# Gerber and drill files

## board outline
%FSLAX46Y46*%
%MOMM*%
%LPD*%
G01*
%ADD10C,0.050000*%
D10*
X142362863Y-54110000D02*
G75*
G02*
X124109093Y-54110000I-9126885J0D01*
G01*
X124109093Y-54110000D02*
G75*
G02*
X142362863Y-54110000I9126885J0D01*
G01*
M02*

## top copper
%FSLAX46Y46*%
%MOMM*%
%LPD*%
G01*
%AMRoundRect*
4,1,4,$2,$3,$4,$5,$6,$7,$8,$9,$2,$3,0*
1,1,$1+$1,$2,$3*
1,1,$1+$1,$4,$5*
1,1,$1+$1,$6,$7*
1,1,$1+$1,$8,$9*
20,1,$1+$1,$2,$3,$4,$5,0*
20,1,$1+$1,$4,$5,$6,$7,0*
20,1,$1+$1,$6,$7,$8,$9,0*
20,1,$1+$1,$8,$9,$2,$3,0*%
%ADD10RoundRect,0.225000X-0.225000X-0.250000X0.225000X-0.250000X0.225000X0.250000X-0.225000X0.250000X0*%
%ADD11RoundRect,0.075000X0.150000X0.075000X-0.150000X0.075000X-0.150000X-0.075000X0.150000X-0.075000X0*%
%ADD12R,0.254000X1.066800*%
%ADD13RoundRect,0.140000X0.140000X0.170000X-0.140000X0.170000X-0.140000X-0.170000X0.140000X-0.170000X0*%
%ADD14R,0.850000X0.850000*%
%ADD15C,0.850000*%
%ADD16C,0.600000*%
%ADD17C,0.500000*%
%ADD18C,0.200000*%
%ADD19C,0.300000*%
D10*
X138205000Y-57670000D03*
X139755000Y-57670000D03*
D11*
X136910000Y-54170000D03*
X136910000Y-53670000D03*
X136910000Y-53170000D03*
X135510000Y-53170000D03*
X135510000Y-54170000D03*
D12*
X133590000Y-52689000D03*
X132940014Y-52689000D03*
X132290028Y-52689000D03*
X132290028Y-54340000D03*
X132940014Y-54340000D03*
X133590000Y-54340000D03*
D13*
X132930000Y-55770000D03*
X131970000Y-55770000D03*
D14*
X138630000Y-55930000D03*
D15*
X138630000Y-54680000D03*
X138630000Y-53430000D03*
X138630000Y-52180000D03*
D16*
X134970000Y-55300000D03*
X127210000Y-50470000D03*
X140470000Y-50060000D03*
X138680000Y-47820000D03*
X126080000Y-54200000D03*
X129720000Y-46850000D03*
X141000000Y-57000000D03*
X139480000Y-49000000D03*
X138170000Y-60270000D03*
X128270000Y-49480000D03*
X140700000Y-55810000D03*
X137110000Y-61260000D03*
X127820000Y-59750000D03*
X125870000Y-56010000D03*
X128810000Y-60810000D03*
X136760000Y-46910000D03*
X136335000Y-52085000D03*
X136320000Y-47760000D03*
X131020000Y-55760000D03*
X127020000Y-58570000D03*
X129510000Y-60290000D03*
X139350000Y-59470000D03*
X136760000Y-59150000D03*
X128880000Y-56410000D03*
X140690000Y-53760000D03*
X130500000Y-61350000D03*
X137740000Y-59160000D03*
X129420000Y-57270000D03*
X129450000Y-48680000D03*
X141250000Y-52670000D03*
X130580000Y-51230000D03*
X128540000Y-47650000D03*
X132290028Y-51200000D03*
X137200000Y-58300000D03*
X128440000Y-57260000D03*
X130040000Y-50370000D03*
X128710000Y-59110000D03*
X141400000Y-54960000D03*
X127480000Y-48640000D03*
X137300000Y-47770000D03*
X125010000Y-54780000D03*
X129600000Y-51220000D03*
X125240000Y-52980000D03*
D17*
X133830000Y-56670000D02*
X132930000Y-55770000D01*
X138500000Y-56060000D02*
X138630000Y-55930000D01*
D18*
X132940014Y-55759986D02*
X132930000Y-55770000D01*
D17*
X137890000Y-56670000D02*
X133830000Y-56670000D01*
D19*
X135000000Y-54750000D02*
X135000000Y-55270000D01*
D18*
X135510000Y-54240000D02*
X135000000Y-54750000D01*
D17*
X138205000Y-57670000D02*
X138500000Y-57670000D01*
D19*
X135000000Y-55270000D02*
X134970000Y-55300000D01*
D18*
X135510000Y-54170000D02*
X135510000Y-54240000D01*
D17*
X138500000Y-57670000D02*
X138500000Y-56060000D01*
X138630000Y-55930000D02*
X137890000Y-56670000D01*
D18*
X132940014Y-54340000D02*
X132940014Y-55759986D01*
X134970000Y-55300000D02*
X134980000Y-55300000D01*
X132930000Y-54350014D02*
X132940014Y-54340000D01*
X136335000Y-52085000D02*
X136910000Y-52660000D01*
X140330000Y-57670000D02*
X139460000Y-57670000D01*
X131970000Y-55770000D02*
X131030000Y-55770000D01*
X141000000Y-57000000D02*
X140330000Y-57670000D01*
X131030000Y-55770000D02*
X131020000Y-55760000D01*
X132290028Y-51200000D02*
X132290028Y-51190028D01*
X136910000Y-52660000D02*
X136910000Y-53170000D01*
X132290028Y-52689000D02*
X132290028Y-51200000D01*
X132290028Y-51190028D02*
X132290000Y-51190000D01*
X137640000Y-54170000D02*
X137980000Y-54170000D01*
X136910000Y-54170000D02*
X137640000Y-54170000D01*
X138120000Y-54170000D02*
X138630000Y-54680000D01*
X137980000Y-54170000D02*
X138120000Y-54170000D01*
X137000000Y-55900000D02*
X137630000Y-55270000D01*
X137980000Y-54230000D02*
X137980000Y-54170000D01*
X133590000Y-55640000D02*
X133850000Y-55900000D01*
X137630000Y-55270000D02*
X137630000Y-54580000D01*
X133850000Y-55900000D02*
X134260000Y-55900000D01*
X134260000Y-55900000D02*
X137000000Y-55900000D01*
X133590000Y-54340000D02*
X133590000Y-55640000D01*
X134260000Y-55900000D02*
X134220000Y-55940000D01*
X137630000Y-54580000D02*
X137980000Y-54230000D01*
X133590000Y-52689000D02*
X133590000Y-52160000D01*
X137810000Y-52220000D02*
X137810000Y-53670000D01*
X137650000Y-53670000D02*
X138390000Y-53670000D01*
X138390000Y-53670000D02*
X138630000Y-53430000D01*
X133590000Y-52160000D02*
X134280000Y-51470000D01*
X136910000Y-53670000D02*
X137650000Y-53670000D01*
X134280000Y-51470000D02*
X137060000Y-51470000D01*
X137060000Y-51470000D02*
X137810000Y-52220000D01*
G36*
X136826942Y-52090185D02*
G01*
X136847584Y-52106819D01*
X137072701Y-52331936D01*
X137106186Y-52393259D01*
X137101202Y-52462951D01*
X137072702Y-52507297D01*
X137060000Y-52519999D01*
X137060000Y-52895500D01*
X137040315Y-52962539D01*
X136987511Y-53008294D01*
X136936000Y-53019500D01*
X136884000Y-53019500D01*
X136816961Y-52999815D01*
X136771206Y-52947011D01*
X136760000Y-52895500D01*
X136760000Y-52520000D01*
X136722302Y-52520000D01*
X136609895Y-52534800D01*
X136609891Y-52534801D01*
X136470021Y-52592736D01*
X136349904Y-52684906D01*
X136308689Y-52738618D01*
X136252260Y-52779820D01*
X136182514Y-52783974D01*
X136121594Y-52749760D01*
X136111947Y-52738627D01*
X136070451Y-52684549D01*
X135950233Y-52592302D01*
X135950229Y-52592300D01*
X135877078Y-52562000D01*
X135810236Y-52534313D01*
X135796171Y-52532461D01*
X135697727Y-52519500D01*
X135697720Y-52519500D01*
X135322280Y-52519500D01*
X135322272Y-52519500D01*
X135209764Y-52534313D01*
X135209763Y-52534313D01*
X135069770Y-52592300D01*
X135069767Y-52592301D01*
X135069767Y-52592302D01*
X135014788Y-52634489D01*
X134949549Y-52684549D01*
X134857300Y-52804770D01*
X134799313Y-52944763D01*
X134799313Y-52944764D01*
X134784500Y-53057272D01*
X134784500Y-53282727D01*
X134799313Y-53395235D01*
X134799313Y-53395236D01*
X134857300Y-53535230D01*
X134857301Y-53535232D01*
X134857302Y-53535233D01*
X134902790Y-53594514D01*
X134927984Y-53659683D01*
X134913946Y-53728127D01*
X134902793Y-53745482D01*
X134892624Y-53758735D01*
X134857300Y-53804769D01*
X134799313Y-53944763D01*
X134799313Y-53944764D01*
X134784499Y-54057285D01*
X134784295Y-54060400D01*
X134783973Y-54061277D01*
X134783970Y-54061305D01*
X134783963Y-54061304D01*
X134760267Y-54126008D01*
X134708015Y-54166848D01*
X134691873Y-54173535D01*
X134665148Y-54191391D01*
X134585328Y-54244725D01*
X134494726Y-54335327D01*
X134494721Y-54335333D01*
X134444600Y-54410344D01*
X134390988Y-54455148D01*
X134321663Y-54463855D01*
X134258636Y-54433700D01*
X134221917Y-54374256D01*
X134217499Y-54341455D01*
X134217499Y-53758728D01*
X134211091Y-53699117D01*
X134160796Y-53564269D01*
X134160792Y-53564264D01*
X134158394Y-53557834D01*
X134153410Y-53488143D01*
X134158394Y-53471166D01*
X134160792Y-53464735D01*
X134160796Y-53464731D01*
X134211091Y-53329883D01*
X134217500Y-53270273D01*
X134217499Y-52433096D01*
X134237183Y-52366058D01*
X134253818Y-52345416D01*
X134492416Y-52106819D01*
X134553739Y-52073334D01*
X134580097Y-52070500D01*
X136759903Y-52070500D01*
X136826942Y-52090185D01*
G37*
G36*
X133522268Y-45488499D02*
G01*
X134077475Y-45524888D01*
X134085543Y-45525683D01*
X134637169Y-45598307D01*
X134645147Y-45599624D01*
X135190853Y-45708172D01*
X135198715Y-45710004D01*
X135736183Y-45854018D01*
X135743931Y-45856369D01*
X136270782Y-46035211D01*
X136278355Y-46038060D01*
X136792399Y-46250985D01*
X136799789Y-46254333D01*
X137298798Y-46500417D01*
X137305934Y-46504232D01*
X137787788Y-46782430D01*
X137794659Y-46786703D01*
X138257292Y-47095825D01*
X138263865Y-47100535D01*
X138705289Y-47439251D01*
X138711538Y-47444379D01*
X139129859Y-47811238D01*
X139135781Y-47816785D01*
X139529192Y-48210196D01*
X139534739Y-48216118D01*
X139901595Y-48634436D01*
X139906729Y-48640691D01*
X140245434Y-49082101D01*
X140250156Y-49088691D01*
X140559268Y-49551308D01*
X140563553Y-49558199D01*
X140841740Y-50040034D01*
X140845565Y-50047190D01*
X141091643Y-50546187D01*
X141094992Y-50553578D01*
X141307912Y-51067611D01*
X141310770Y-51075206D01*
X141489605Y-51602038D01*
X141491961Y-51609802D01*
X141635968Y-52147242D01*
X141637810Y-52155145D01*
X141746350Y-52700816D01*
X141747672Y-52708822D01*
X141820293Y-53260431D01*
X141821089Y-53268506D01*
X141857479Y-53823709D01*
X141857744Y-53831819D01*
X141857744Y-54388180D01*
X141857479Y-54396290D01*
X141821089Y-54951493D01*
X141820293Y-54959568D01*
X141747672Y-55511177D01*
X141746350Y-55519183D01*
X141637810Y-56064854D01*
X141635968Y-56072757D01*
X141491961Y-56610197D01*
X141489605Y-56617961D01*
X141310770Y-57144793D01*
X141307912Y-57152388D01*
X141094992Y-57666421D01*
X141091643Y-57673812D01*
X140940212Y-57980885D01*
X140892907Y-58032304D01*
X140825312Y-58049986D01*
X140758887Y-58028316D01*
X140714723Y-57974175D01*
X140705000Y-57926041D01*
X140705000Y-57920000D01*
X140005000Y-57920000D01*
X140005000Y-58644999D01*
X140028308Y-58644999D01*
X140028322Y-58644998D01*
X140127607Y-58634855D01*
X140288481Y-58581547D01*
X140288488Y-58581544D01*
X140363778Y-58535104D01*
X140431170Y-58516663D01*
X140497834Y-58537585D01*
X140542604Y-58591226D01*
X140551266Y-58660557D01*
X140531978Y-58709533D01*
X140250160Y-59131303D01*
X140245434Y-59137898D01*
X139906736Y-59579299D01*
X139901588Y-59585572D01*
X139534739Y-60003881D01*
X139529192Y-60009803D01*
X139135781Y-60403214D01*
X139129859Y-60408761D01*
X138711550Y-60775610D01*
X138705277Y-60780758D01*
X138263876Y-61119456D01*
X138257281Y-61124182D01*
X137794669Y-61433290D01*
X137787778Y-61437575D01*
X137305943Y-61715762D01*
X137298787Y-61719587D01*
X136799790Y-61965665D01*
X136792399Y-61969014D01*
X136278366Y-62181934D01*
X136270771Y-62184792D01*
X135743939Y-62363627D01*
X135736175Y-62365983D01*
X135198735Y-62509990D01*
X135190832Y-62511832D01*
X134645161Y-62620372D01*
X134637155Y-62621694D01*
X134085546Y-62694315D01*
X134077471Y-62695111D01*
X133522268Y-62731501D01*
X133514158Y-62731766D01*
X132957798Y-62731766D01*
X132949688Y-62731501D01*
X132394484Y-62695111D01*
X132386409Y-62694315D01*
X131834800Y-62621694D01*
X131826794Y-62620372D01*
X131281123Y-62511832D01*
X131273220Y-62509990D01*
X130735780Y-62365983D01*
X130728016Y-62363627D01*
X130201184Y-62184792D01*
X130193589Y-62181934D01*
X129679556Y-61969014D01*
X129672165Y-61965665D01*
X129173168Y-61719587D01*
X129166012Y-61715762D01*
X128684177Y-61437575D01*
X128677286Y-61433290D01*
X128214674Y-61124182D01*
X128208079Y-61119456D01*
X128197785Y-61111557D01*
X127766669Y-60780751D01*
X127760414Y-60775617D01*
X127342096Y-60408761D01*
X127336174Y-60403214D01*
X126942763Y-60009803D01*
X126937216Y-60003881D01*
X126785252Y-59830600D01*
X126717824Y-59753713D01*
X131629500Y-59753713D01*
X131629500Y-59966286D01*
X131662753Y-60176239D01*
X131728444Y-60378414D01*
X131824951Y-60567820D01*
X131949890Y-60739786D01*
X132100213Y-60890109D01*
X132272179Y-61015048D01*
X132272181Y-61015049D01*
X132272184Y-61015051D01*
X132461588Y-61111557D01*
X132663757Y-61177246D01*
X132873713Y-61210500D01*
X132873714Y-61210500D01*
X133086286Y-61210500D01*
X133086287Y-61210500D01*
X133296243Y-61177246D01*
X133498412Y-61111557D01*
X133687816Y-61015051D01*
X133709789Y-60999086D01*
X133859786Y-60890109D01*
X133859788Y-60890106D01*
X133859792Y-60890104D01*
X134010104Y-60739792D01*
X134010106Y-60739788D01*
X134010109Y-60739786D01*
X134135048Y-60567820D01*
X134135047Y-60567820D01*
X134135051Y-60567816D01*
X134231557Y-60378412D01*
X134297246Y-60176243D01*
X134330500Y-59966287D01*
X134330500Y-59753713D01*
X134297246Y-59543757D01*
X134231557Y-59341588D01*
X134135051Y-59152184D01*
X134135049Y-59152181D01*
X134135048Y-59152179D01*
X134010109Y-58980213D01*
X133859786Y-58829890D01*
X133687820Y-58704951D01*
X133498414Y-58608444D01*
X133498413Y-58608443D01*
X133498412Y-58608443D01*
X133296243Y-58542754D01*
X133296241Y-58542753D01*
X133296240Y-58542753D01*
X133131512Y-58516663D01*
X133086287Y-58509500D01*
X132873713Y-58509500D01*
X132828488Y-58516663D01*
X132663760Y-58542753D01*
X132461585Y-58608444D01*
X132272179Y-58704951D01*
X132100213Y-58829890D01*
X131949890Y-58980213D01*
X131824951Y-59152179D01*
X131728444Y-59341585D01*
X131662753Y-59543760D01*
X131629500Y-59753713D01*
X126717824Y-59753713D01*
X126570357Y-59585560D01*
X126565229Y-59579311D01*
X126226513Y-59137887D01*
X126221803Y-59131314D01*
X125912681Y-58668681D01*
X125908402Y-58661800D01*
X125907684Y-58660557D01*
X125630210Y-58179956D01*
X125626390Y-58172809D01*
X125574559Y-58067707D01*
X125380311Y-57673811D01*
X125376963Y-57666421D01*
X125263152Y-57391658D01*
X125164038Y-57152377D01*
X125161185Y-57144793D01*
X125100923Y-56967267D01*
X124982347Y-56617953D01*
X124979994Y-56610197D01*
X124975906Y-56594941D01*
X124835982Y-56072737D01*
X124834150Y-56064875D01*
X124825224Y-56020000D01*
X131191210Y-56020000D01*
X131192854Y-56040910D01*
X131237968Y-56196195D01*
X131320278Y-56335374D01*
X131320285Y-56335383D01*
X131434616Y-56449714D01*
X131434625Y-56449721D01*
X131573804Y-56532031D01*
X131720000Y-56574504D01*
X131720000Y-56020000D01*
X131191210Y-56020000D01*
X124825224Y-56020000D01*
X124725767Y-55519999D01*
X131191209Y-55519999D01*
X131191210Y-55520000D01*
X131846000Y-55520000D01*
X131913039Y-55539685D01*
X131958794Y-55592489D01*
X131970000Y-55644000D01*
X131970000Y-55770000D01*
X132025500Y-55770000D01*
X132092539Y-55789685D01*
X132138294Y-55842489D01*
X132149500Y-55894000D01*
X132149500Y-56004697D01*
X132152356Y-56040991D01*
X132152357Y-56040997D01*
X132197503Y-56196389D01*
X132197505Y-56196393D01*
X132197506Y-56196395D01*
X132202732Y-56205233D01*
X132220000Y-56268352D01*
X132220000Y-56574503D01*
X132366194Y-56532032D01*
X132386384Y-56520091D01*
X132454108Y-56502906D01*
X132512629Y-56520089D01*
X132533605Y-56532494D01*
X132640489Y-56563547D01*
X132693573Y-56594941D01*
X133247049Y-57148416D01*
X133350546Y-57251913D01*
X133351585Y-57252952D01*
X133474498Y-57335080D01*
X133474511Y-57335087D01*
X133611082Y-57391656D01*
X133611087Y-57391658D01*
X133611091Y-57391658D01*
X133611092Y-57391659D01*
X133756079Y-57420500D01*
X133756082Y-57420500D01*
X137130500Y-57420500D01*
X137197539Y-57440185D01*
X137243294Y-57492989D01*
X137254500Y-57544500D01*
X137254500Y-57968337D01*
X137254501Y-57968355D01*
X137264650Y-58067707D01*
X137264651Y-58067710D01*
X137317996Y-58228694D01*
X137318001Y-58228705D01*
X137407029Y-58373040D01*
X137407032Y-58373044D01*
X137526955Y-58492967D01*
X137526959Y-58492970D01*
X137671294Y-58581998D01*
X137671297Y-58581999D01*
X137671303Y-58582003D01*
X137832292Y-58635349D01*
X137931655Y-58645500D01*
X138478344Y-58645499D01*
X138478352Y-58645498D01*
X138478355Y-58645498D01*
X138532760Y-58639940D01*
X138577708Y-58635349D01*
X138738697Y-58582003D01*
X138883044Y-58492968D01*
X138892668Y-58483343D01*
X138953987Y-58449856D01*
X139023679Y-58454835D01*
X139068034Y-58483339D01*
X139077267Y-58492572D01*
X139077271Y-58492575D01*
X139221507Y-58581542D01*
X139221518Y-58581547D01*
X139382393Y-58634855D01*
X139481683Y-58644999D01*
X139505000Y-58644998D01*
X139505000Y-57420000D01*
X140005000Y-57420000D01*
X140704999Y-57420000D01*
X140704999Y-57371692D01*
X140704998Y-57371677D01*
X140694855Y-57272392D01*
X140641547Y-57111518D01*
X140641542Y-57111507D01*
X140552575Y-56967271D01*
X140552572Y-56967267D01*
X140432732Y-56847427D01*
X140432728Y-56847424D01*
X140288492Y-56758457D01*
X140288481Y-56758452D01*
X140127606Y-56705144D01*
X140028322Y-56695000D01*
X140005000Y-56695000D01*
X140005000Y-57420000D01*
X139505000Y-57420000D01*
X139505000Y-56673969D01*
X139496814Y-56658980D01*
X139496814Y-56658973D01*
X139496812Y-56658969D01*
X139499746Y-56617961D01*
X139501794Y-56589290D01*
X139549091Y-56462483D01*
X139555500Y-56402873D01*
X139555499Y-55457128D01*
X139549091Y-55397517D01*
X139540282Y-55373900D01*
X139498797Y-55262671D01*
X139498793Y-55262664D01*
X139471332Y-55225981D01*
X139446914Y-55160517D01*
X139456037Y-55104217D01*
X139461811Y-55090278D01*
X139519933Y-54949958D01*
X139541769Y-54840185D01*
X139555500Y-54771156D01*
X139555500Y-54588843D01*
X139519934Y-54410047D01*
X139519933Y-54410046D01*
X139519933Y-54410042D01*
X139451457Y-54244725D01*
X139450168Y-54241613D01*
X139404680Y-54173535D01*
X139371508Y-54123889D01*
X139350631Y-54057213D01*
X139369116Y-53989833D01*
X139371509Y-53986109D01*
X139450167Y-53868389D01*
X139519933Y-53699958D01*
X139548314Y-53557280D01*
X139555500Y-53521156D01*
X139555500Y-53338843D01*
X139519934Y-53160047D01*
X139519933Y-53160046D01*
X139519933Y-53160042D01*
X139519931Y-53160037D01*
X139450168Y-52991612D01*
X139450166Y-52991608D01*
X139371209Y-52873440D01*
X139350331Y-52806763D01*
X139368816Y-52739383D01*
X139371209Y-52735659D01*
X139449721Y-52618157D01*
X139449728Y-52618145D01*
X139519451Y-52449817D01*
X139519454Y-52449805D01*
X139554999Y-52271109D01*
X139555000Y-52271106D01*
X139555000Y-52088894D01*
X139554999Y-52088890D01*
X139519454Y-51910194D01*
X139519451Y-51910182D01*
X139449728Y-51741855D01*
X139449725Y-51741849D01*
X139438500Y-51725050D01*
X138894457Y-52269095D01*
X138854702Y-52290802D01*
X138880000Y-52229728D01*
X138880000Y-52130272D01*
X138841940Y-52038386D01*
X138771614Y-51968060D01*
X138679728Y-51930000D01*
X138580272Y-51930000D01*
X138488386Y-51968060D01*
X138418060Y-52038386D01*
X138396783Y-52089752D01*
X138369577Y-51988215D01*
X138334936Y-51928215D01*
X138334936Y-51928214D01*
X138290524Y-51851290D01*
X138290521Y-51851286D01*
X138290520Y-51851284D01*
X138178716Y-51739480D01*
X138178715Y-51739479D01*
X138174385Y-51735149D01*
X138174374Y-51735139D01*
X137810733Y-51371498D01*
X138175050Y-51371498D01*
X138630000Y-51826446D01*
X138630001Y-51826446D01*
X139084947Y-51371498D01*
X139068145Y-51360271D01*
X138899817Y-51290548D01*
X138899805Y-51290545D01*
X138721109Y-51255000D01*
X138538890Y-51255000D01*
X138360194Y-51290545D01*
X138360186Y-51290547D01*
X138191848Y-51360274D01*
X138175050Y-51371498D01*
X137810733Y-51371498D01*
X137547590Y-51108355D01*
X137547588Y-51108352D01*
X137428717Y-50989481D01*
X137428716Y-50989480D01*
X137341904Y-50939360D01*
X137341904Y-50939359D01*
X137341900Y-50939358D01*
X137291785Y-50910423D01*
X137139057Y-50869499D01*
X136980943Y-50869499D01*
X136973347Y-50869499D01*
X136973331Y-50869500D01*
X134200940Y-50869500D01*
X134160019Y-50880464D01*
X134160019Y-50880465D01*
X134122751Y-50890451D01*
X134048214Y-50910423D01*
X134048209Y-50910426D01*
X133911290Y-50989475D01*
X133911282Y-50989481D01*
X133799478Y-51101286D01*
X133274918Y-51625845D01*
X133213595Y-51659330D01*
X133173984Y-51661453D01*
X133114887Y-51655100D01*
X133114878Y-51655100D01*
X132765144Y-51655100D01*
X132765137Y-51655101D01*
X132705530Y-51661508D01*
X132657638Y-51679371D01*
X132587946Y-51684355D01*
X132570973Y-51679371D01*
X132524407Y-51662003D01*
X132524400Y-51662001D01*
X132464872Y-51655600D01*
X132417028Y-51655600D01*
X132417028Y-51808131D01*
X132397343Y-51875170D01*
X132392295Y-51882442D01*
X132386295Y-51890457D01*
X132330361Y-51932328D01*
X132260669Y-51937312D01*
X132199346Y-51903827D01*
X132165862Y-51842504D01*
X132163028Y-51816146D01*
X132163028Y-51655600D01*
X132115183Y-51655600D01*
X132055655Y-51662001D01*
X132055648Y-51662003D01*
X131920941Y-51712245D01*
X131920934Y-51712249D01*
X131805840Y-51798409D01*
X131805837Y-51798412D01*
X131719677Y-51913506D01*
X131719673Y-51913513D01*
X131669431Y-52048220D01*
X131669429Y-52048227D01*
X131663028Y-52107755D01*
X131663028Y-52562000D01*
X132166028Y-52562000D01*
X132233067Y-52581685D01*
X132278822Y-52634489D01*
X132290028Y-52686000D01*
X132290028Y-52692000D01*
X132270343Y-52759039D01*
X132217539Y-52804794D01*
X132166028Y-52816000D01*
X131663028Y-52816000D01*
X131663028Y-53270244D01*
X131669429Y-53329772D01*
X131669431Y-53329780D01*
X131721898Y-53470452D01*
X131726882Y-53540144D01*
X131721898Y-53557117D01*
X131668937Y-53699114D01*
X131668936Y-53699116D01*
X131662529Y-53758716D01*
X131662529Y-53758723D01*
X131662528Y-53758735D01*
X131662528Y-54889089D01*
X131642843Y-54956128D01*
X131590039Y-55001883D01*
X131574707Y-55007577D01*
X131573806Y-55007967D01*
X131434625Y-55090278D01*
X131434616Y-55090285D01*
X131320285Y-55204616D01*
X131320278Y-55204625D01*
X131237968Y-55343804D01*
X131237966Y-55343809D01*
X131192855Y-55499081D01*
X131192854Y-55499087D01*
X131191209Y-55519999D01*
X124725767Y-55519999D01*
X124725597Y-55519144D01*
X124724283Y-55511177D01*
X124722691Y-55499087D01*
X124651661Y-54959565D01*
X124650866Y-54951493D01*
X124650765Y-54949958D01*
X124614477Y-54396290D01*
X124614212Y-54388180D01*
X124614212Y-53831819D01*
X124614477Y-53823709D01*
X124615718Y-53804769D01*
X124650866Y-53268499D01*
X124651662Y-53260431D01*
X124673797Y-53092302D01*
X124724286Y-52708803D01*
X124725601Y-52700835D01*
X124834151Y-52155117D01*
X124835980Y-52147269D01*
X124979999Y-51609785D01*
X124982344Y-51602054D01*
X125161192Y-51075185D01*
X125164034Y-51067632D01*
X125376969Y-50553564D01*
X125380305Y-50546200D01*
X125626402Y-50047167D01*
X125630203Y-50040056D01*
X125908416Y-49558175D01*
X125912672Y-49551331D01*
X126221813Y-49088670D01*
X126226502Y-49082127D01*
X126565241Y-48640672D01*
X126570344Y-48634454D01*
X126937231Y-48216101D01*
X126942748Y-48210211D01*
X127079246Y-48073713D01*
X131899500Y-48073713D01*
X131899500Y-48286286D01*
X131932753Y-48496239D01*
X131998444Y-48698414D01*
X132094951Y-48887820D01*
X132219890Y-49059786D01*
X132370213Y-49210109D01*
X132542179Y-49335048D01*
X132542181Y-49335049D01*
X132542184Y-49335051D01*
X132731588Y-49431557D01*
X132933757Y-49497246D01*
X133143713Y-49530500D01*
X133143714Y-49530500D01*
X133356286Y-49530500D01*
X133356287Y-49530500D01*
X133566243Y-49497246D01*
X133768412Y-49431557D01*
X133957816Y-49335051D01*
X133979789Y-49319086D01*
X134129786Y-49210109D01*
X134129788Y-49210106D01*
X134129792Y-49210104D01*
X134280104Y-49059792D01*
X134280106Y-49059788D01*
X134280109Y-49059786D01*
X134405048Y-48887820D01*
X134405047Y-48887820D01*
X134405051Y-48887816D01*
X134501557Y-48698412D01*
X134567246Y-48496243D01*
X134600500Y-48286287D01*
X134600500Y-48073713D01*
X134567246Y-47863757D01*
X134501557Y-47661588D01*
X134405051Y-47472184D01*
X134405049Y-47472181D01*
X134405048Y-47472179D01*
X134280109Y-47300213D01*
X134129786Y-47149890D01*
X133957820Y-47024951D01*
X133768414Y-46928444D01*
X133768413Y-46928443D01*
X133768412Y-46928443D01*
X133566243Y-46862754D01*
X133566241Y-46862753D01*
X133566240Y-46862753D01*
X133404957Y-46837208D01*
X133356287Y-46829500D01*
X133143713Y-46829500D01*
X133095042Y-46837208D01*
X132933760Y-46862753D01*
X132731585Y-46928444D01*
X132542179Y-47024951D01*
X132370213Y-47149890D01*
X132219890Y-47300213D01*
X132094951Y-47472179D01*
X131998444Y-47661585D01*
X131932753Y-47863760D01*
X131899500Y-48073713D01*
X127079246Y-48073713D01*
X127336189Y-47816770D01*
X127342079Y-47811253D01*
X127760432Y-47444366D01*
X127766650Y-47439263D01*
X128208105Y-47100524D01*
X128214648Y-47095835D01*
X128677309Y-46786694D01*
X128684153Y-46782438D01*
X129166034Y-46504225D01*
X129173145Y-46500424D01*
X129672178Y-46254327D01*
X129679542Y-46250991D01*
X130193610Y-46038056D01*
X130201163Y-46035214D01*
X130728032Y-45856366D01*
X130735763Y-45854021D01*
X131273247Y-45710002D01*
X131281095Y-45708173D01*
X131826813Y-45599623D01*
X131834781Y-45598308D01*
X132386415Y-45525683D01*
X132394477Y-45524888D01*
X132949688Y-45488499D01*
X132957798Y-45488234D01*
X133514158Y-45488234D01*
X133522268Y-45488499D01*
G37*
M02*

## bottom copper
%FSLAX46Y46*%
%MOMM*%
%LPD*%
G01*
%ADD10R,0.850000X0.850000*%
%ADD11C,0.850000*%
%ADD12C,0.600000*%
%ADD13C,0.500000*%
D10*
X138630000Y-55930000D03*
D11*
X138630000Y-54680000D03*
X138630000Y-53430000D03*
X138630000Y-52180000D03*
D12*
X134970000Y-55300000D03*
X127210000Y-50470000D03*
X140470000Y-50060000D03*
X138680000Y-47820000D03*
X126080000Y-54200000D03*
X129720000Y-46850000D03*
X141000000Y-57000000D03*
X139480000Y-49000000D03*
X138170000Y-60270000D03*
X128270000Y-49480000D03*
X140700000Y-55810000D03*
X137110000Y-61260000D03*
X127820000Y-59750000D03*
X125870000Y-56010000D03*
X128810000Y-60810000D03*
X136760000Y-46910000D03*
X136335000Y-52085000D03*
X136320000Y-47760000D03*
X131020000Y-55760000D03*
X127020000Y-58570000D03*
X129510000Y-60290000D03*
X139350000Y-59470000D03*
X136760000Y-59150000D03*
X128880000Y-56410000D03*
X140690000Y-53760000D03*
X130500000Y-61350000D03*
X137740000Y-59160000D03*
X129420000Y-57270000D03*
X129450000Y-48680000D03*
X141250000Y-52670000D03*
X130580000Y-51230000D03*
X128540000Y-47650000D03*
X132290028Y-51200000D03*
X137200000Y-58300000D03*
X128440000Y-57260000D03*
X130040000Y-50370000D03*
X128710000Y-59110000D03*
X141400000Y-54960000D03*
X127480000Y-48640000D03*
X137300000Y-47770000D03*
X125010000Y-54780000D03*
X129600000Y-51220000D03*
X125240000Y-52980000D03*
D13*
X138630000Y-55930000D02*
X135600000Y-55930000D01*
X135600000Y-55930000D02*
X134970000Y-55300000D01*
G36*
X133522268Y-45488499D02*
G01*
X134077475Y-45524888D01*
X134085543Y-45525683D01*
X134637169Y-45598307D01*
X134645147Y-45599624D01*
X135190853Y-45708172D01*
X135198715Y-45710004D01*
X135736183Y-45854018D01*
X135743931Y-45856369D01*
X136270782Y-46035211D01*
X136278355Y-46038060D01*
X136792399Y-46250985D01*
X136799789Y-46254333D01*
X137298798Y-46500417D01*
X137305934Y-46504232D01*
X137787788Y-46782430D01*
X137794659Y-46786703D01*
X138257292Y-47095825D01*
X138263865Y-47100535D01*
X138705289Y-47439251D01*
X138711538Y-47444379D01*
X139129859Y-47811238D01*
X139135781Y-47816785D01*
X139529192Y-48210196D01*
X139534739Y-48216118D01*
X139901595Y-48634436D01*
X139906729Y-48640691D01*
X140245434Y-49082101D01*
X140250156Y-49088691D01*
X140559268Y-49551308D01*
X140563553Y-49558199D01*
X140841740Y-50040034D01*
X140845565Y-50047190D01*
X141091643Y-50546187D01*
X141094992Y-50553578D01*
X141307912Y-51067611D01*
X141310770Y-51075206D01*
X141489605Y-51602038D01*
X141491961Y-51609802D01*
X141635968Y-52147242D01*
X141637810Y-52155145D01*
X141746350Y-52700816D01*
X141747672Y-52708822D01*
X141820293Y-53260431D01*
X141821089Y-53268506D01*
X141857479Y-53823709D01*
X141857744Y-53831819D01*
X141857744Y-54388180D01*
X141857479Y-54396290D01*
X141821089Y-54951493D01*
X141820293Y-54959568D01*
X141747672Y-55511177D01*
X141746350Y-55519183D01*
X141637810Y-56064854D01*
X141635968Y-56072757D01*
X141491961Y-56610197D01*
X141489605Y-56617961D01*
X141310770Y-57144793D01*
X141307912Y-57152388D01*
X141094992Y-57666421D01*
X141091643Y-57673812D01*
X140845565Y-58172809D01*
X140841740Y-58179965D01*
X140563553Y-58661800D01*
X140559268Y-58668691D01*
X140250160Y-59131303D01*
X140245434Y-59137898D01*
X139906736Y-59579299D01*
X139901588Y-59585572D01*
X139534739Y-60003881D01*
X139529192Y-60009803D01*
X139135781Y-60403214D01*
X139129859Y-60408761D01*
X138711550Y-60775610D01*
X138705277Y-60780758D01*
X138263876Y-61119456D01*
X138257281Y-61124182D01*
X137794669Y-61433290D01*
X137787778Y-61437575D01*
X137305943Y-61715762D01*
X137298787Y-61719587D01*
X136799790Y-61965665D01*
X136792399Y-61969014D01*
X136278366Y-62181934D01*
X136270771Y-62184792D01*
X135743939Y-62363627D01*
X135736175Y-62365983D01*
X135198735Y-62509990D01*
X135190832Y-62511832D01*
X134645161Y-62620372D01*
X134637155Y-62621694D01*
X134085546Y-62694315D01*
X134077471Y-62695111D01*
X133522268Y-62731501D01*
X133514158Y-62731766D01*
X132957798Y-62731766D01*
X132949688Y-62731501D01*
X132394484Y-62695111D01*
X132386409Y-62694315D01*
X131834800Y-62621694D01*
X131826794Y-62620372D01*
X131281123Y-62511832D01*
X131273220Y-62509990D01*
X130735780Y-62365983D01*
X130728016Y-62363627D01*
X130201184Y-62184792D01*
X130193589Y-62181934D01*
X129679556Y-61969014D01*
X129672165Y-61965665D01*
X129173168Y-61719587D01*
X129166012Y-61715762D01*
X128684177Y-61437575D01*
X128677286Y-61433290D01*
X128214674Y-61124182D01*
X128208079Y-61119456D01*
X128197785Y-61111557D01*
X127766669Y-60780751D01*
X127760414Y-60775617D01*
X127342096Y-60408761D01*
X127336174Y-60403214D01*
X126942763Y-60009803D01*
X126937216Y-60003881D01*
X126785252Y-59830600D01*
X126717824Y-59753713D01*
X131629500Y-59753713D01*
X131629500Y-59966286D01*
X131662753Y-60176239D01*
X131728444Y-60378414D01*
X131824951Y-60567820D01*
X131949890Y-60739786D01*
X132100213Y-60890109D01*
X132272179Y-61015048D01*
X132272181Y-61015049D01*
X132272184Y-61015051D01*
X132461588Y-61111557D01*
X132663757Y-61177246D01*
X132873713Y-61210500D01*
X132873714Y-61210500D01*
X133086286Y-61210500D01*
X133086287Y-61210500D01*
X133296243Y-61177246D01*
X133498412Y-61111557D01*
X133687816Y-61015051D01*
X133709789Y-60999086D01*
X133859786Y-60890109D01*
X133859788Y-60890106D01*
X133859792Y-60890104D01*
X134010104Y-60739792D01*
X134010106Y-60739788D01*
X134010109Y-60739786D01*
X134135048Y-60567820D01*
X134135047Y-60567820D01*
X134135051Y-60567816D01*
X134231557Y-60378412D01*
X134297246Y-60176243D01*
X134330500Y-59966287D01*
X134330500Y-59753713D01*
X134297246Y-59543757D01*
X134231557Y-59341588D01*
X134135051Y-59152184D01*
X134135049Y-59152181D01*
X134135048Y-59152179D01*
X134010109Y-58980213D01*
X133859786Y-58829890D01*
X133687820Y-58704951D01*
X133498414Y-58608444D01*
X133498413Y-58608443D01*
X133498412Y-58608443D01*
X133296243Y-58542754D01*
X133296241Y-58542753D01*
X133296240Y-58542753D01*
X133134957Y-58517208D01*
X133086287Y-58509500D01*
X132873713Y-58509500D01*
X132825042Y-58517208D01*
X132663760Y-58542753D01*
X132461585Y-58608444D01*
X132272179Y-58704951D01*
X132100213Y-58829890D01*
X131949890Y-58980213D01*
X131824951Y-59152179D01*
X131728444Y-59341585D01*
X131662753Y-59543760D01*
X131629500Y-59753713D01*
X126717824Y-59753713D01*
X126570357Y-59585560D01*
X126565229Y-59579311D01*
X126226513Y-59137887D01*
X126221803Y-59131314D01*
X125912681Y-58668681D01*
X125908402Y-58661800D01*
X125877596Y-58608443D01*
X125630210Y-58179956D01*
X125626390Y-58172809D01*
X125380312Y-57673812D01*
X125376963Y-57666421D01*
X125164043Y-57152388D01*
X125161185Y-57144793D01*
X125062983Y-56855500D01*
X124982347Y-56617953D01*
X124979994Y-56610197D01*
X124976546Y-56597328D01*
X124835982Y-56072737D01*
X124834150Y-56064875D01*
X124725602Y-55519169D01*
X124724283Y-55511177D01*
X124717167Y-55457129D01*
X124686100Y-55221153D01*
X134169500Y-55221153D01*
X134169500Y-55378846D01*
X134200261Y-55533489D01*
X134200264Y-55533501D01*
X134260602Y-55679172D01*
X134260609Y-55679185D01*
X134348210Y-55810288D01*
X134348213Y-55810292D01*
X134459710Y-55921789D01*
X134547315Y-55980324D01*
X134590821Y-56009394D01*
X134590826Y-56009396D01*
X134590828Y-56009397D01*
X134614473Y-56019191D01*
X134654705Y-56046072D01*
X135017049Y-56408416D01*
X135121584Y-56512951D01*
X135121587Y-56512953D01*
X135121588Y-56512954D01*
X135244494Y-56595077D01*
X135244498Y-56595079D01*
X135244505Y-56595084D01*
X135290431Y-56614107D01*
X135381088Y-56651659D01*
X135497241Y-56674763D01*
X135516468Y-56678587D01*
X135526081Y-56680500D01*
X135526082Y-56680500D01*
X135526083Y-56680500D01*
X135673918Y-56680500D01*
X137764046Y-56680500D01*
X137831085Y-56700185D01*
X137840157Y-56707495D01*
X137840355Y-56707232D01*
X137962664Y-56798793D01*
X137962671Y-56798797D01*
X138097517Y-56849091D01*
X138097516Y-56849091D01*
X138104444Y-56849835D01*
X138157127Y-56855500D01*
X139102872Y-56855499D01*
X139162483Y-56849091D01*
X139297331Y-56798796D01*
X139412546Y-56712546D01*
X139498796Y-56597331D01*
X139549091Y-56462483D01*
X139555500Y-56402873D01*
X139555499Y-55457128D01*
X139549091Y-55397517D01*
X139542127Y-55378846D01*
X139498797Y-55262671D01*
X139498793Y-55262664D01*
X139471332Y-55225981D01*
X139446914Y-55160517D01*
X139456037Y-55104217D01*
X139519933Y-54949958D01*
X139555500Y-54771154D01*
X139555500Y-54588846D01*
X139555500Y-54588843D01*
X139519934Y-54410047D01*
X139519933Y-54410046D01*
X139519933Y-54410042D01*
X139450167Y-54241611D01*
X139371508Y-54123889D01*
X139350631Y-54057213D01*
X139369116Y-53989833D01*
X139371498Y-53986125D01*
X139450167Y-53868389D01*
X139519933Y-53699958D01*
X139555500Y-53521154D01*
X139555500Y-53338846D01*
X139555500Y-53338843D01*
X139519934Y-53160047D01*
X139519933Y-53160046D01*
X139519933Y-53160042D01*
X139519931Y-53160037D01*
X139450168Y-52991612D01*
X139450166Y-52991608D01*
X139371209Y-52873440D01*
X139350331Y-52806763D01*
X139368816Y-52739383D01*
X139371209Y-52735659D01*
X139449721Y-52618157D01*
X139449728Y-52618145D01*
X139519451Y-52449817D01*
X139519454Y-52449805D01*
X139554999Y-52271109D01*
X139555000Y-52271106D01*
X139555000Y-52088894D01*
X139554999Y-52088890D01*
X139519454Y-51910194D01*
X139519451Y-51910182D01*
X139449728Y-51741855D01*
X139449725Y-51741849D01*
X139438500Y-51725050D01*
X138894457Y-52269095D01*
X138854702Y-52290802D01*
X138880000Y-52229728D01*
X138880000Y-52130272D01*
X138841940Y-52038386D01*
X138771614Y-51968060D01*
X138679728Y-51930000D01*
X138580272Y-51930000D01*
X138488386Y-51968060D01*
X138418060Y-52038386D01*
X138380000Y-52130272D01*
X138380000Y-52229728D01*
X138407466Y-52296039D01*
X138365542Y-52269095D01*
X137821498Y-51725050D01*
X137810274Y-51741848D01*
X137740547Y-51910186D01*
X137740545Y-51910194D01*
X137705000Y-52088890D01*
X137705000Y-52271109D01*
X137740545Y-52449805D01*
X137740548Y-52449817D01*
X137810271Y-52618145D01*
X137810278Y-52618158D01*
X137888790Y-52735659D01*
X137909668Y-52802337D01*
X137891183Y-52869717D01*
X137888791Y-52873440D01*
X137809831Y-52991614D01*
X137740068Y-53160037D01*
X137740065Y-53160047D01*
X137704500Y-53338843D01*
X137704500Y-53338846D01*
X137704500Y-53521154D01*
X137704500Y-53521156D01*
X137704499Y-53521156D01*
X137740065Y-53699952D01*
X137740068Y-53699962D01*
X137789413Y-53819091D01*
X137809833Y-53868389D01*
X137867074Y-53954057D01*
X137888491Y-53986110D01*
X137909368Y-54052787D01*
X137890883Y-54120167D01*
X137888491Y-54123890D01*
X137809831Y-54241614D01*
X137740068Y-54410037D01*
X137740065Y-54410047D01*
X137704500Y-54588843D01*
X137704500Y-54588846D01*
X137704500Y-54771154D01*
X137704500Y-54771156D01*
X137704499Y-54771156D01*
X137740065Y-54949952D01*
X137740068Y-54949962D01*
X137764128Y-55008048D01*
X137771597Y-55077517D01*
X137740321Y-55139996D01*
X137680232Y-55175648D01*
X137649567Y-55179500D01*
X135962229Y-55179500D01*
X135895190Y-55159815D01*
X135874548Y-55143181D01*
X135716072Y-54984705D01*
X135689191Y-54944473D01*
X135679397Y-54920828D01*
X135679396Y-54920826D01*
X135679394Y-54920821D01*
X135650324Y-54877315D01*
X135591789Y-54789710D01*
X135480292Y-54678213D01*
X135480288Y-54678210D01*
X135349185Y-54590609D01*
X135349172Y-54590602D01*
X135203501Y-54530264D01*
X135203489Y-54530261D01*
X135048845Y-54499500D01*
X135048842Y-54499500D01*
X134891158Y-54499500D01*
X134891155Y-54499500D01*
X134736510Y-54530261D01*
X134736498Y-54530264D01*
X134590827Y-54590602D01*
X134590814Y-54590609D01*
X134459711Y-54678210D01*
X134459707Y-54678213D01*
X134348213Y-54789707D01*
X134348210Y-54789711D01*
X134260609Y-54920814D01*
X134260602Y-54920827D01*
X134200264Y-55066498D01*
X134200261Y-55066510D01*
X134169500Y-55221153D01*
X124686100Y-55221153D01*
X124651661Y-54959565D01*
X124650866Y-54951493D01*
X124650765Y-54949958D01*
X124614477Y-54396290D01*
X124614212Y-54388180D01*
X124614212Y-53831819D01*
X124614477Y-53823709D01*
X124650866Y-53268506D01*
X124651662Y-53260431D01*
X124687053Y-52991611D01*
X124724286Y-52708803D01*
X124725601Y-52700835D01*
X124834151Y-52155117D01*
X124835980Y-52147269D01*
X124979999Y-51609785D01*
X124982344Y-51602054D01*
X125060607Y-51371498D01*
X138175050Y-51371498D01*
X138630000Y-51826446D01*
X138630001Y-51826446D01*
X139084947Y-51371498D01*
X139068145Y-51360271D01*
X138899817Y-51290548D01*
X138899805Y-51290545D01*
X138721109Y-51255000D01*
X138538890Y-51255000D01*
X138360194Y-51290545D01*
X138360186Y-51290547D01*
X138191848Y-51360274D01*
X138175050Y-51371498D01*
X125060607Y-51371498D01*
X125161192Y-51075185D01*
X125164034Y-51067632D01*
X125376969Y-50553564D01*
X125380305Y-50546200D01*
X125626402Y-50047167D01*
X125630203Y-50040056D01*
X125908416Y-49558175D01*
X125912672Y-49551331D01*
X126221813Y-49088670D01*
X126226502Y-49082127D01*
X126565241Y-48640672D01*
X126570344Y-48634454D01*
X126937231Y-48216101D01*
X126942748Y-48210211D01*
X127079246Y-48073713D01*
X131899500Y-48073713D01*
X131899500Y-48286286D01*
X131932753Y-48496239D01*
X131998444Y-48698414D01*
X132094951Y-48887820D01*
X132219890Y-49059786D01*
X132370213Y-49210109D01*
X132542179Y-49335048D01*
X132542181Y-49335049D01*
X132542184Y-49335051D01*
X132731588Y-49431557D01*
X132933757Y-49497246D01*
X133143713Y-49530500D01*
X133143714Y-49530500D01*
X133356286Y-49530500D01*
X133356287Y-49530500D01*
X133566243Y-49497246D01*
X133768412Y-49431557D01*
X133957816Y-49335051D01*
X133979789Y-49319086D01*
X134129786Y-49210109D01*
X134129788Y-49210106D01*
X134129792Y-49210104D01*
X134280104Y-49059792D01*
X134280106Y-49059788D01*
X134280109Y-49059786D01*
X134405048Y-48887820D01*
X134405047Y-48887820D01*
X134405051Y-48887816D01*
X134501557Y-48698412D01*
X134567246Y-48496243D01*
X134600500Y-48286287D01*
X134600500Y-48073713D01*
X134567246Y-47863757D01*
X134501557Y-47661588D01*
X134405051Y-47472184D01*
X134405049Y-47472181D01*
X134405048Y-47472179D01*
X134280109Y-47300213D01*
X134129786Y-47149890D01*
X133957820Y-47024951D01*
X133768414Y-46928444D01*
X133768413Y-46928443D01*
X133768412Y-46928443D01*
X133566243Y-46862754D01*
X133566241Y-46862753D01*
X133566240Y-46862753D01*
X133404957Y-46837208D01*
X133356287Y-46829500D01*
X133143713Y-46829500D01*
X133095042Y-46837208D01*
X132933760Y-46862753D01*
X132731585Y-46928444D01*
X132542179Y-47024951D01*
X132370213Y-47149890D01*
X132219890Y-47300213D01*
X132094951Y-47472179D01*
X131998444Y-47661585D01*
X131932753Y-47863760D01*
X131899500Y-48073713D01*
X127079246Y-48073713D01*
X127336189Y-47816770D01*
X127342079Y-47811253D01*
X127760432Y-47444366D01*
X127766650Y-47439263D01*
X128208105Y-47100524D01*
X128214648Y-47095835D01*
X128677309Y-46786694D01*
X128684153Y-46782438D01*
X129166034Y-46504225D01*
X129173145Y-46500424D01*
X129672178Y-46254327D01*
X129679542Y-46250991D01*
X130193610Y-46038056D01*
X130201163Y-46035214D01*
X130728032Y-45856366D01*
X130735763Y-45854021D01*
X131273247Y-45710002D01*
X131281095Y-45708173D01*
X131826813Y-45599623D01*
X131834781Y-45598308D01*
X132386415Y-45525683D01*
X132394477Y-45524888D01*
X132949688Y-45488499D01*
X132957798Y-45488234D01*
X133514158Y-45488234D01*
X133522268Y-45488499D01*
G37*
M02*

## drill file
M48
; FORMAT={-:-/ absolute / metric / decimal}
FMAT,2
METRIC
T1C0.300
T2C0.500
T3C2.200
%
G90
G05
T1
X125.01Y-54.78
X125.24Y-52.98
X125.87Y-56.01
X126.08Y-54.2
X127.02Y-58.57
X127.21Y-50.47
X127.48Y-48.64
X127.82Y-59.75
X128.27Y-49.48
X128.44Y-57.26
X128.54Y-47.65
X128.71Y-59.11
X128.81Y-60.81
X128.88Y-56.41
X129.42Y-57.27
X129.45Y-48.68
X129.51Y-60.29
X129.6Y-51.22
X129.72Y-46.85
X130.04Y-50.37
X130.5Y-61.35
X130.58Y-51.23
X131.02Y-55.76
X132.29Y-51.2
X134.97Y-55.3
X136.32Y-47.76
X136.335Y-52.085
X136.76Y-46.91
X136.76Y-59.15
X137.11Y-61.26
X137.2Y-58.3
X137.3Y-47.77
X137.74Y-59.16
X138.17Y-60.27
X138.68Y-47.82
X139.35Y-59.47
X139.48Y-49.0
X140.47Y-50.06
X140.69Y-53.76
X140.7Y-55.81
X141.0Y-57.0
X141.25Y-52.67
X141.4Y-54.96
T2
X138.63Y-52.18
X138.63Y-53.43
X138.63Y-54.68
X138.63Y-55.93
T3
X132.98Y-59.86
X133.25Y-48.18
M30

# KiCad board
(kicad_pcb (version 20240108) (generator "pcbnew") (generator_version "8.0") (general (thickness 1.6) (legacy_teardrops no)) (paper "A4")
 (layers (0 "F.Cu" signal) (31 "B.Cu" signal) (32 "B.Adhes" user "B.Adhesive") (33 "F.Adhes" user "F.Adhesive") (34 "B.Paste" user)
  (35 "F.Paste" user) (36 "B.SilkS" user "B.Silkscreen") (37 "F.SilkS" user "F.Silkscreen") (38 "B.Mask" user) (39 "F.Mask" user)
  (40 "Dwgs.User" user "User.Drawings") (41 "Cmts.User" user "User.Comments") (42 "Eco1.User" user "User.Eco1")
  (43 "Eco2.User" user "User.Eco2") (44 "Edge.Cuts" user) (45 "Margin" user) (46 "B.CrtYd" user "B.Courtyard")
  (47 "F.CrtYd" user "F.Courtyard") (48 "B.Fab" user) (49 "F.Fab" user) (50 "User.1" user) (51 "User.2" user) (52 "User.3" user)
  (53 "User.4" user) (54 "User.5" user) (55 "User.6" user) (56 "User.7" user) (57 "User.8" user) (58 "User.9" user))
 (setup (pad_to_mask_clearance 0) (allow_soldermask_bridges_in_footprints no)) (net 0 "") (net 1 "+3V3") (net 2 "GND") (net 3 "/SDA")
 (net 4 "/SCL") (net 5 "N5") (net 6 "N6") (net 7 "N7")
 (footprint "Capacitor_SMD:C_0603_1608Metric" (layer "F.Cu") (at 138.98 57.67)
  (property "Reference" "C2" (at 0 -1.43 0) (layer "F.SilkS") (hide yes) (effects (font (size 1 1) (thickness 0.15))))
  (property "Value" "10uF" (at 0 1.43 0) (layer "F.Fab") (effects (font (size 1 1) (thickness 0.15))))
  (pad "1" smd roundrect (at -0.775 0) (size 0.9 0.95) (layers "F.Cu" "F.Paste" "F.Mask") (roundrect_rratio 0.25) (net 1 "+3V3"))
  (pad "2" smd roundrect (at 0.775 0) (size 0.9 0.95) (layers "F.Cu" "F.Paste" "F.Mask") (roundrect_rratio 0.25) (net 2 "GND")))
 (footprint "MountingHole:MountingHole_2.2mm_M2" (layer "F.Cu") (at 132.98 59.86)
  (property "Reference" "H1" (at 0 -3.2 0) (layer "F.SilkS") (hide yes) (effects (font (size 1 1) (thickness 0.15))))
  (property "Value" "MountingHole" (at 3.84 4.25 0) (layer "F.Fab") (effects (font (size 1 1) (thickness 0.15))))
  (pad "" np_thru_hole circle (at 0 0) (size 2.2 2.2) (drill 2.2) (layers "*.Cu" "*.Mask")))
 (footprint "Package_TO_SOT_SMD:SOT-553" (layer "F.Cu") (at 136.21 53.67 180)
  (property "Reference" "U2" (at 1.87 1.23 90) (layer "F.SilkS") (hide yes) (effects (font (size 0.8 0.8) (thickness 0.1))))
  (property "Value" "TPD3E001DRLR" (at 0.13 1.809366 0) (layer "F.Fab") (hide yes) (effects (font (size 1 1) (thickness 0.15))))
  (pad "1" smd roundrect (at -0.7 -0.5 180) (size 0.45 0.3) (layers "F.Cu" "F.Paste" "F.Mask") (roundrect_rratio 0.25) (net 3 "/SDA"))
  (pad "2" smd roundrect (at -0.7 0 180) (size 0.45 0.3) (layers "F.Cu" "F.Paste" "F.Mask") (roundrect_rratio 0.25) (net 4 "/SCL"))
  (pad "3" smd roundrect (at -0.7 0.5 180) (size 0.45 0.3) (layers "F.Cu" "F.Paste" "F.Mask") (roundrect_rratio 0.25) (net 2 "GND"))
  (pad "4" smd roundrect (at 0.7 0.5 180) (size 0.45 0.3) (layers "F.Cu" "F.Paste" "F.Mask") (roundrect_rratio 0.25) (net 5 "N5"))
  (pad "5" smd roundrect (at 0.7 -0.5 180) (size 0.45 0.3) (layers "F.Cu" "F.Paste" "F.Mask") (roundrect_rratio 0.25) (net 1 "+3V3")))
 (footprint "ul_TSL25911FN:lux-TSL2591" (layer "F.Cu") (at 132.940014 53.5145 -90)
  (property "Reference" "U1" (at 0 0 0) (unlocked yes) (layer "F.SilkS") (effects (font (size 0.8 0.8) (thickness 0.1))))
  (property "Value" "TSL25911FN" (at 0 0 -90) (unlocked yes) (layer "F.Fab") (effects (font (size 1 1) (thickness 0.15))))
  (pad "1" smd rect (at -0.8255 -0.649986 270) (size 1.0668 0.254) (layers "F.Cu" "F.Paste" "F.Mask") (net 4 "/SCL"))
  (pad "2" smd rect (at -0.8255 0 270) (size 1.0668 0.254) (layers "F.Cu" "F.Paste" "F.Mask") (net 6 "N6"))
  (pad "3" smd rect (at -0.8255 0.649986 270) (size 1.0668 0.254) (layers "F.Cu" "F.Paste" "F.Mask") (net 2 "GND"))
  (pad "4" smd rect (at 0.8255 0.649986 270) (size 1.0668 0.254) (layers "F.Cu" "F.Paste" "F.Mask") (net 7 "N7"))
  (pad "5" smd rect (at 0.8255 0 270) (size 1.0668 0.254) (layers "F.Cu" "F.Paste" "F.Mask") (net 1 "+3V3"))
  (pad "6" smd rect (at 0.8255 -0.649986 270) (size 1.0668 0.254) (layers "F.Cu" "F.Paste" "F.Mask") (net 3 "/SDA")))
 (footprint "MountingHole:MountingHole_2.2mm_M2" (layer "F.Cu") (at 133.25 48.18)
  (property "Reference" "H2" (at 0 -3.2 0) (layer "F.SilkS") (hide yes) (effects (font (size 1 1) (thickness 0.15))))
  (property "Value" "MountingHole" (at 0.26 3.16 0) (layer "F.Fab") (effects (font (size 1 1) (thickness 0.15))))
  (pad "" np_thru_hole circle (at 0 0) (size 2.2 2.2) (drill 2.2) (layers "*.Cu" "*.Mask")))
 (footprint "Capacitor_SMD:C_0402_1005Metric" (layer "F.Cu") (at 132.45 55.77 180)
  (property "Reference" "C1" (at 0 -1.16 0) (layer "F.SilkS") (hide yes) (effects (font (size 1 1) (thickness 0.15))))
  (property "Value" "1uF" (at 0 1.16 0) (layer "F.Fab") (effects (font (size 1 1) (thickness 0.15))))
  (pad "1" smd roundrect (at -0.48 0 180) (size 0.56 0.62) (layers "F.Cu" "F.Paste" "F.Mask") (roundrect_rratio 0.25) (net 1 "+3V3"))
  (pad "2" smd roundrect (at 0.48 0 180) (size 0.56 0.62) (layers "F.Cu" "F.Paste" "F.Mask") (roundrect_rratio 0.25) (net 2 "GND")))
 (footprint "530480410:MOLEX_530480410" (layer "B.Cu") (at 138.63 55.93 90)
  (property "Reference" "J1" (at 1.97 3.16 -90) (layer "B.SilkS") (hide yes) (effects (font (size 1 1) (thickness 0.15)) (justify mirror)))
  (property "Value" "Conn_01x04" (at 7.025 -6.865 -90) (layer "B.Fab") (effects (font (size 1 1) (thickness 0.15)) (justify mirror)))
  (pad "1" thru_hole rect (at 0 0 90) (size 0.85 0.85) (drill 0.5) (layers "*.Cu") (remove_unused_layers no) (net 1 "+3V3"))
  (pad "2" thru_hole circle (at 1.25 0 90) (size 0.85 0.85) (drill 0.5) (layers "*.Cu") (remove_unused_layers no) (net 3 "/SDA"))
  (pad "3" thru_hole circle (at 2.5 0 90) (size 0.85 0.85) (drill 0.5) (layers "*.Cu") (remove_unused_layers no) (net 4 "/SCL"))
  (pad "4" thru_hole circle (at 3.75 0 90) (size 0.85 0.85) (drill 0.5) (layers "*.Cu") (remove_unused_layers no) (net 2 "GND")))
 (gr_circle (center 133.235978 54.11) (end 140.34 59.84) (stroke (width 0.05) (type default)) (fill none) (layer "Edge.Cuts"))
 (segment (start 133.83 56.67) (end 132.93 55.77) (width 0.5) (layer "F.Cu") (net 1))
 (segment (start 138.5 56.06) (end 138.63 55.93) (width 0.5) (layer "F.Cu") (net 1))
 (segment (start 132.940014 55.759986) (end 132.93 55.77) (width 0.2) (layer "F.Cu") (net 1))
 (segment (start 137.89 56.67) (end 133.83 56.67) (width 0.5) (layer "F.Cu") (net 1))
 (segment (start 135 54.75) (end 135 55.27) (width 0.3) (layer "F.Cu") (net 1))
 (segment (start 135.51 54.24) (end 135 54.75) (width 0.2) (layer "F.Cu") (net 1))
 (segment (start 138.205 57.67) (end 138.5 57.67) (width 0.5) (layer "F.Cu") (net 1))
 (segment (start 135 55.27) (end 134.97 55.3) (width 0.3) (layer "F.Cu") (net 1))
 (segment (start 135.51 54.17) (end 135.51 54.24) (width 0.2) (layer "F.Cu") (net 1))
 (segment (start 138.5 57.67) (end 138.5 56.06) (width 0.5) (layer "F.Cu") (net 1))
 (segment (start 138.63 55.93) (end 137.89 56.67) (width 0.5) (layer "F.Cu") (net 1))
 (segment (start 132.940014 54.34) (end 132.940014 55.759986) (width 0.2) (layer "F.Cu") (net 1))
 (segment (start 134.97 55.3) (end 134.98 55.3) (width 0.2) (layer "F.Cu") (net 1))
 (segment (start 132.93 54.350014) (end 132.940014 54.34) (width 0.2) (layer "F.Cu") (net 1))
 (via (at 134.97 55.3) (size 0.6) (drill 0.3) (layers "F.Cu" "B.Cu") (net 1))
 (segment (start 138.63 55.93) (end 135.6 55.93) (width 0.5) (layer "B.Cu") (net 1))
 (segment (start 135.6 55.93) (end 134.97 55.3) (width 0.5) (layer "B.Cu") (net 1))
 (segment (start 136.335 52.085) (end 136.91 52.66) (width 0.2) (layer "F.Cu") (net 2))
 (segment (start 140.33 57.67) (end 139.46 57.67) (width 0.2) (layer "F.Cu") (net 2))
 (segment (start 131.97 55.77) (end 131.03 55.77) (width 0.2) (layer "F.Cu") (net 2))
 (segment (start 141 57) (end 140.33 57.67) (width 0.2) (layer "F.Cu") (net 2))
 (segment (start 131.03 55.77) (end 131.02 55.76) (width 0.2) (layer "F.Cu") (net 2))
 (segment (start 132.290028 51.2) (end 132.290028 51.190028) (width 0.2) (layer "F.Cu") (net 2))
 (segment (start 136.91 52.66) (end 136.91 53.17) (width 0.2) (layer "F.Cu") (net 2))
 (segment (start 132.290028 52.689) (end 132.290028 51.2) (width 0.2) (layer "F.Cu") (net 2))
 (segment (start 132.290028 51.190028) (end 132.29 51.19) (width 0.2) (layer "F.Cu") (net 2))
 (via (at 127.21 50.47) (size 0.6) (drill 0.3) (layers "F.Cu" "B.Cu") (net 2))
 (via (at 140.47 50.06) (size 0.6) (drill 0.3) (layers "F.Cu" "B.Cu") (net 2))
 (via (at 138.68 47.82) (size 0.6) (drill 0.3) (layers "F.Cu" "B.Cu") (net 2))
 (via (at 126.08 54.2) (size 0.6) (drill 0.3) (layers "F.Cu" "B.Cu") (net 2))
 (via (at 129.72 46.85) (size 0.6) (drill 0.3) (layers "F.Cu" "B.Cu") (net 2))
 (via (at 141 57) (size 0.6) (drill 0.3) (layers "F.Cu" "B.Cu") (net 2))
 (via (at 139.48 49) (size 0.6) (drill 0.3) (layers "F.Cu" "B.Cu") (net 2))
 (via (at 138.17 60.27) (size 0.6) (drill 0.3) (layers "F.Cu" "B.Cu") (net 2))
 (via (at 128.27 49.48) (size 0.6) (drill 0.3) (layers "F.Cu" "B.Cu") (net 2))
 (via (at 140.7 55.81) (size 0.6) (drill 0.3) (layers "F.Cu" "B.Cu") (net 2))
 (via (at 137.11 61.26) (size 0.6) (drill 0.3) (layers "F.Cu" "B.Cu") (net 2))
 (via (at 127.82 59.75) (size 0.6) (drill 0.3) (layers "F.Cu" "B.Cu") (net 2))
 (via (at 125.87 56.01) (size 0.6) (drill 0.3) (layers "F.Cu" "B.Cu") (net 2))
 (via (at 128.81 60.81) (size 0.6) (drill 0.3) (layers "F.Cu" "B.Cu") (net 2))
 (via (at 136.76 46.91) (size 0.6) (drill 0.3) (layers "F.Cu" "B.Cu") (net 2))
 (via (at 136.335 52.085) (size 0.6) (drill 0.3) (layers "F.Cu" "B.Cu") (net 2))
 (via (at 136.32 47.76) (size 0.6) (drill 0.3) (layers "F.Cu" "B.Cu") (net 2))
 (via (at 131.02 55.76) (size 0.6) (drill 0.3) (layers "F.Cu" "B.Cu") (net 2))
 (via (at 127.02 58.57) (size 0.6) (drill 0.3) (layers "F.Cu" "B.Cu") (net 2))
 (via (at 129.51 60.29) (size 0.6) (drill 0.3) (layers "F.Cu" "B.Cu") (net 2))
 (via (at 139.35 59.47) (size 0.6) (drill 0.3) (layers "F.Cu" "B.Cu") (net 2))
 (via (at 136.76 59.15) (size 0.6) (drill 0.3) (layers "F.Cu" "B.Cu") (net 2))
 (via (at 128.88 56.41) (size 0.6) (drill 0.3) (layers "F.Cu" "B.Cu") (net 2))
 (via (at 140.69 53.76) (size 0.6) (drill 0.3) (layers "F.Cu" "B.Cu") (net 2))
 (via (at 130.5 61.35) (size 0.6) (drill 0.3) (layers "F.Cu" "B.Cu") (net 2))
 (via (at 137.74 59.16) (size 0.6) (drill 0.3) (layers "F.Cu" "B.Cu") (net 2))
 (via (at 129.42 57.27) (size 0.6) (drill 0.3) (layers "F.Cu" "B.Cu") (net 2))
 (via (at 129.45 48.68) (size 0.6) (drill 0.3) (layers "F.Cu" "B.Cu") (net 2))
 (via (at 141.25 52.67) (size 0.6) (drill 0.3) (layers "F.Cu" "B.Cu") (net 2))
 (via (at 130.58 51.23) (size 0.6) (drill 0.3) (layers "F.Cu" "B.Cu") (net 2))
 (via (at 128.54 47.65) (size 0.6) (drill 0.3) (layers "F.Cu" "B.Cu") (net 2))
 (via (at 132.290028 51.2) (size 0.6) (drill 0.3) (layers "F.Cu" "B.Cu") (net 2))
 (via (at 137.2 58.3) (size 0.6) (drill 0.3) (layers "F.Cu" "B.Cu") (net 2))
 (via (at 128.44 57.26) (size 0.6) (drill 0.3) (layers "F.Cu" "B.Cu") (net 2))
 (via (at 130.04 50.37) (size 0.6) (drill 0.3) (layers "F.Cu" "B.Cu") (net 2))
 (via (at 128.71 59.11) (size 0.6) (drill 0.3) (layers "F.Cu" "B.Cu") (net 2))
 (via (at 141.4 54.96) (size 0.6) (drill 0.3) (layers "F.Cu" "B.Cu") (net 2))
 (via (at 127.48 48.64) (size 0.6) (drill 0.3) (layers "F.Cu" "B.Cu") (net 2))
 (via (at 137.3 47.77) (size 0.6) (drill 0.3) (layers "F.Cu" "B.Cu") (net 2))
 (via (at 125.01 54.78) (size 0.6) (drill 0.3) (layers "F.Cu" "B.Cu") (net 2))
 (via (at 129.6 51.22) (size 0.6) (drill 0.3) (layers "F.Cu" "B.Cu") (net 2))
 (via (at 125.24 52.98) (size 0.6) (drill 0.3) (layers "F.Cu" "B.Cu") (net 2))
 (segment (start 137.64 54.17) (end 137.98 54.17) (width 0.2) (layer "F.Cu") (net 3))
 (segment (start 136.91 54.17) (end 137.64 54.17) (width 0.2) (layer "F.Cu") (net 3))
 (segment (start 138.12 54.17) (end 138.63 54.68) (width 0.2) (layer "F.Cu") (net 3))
 (segment (start 137.98 54.17) (end 138.12 54.17) (width 0.2) (layer "F.Cu") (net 3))
 (segment (start 137 55.9) (end 137.63 55.27) (width 0.2) (layer "F.Cu") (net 3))
 (segment (start 137.98 54.23) (end 137.98 54.17) (width 0.2) (layer "F.Cu") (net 3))
 (segment (start 133.59 55.64) (end 133.85 55.9) (width 0.2) (layer "F.Cu") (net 3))
 (segment (start 137.63 55.27) (end 137.63 54.58) (width 0.2) (layer "F.Cu") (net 3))
 (segment (start 133.85 55.9) (end 134.26 55.9) (width 0.2) (layer "F.Cu") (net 3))
 (segment (start 134.26 55.9) (end 137 55.9) (width 0.2) (layer "F.Cu") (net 3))
 (segment (start 133.59 54.34) (end 133.59 55.64) (width 0.2) (layer "F.Cu") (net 3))
 (segment (start 134.26 55.9) (end 134.22 55.94) (width 0.2) (layer "F.Cu") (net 3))
 (segment (start 137.63 54.58) (end 137.98 54.23) (width 0.2) (layer "F.Cu") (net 3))
 (segment (start 133.59 52.689) (end 133.59 52.16) (width 0.2) (layer "F.Cu") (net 4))
 (segment (start 137.81 52.22) (end 137.81 53.67) (width 0.2) (layer "F.Cu") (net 4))
 (segment (start 137.65 53.67) (end 138.39 53.67) (width 0.2) (layer "F.Cu") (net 4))
 (segment (start 138.39 53.67) (end 138.63 53.43) (width 0.2) (layer "F.Cu") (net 4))
 (segment (start 133.59 52.16) (end 134.28 51.47) (width 0.2) (layer "F.Cu") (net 4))
 (segment (start 136.91 53.67) (end 137.65 53.67) (width 0.2) (layer "F.Cu") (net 4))
 (segment (start 134.28 51.47) (end 137.06 51.47) (width 0.2) (layer "F.Cu") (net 4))
 (segment (start 137.06 51.47) (end 137.81 52.22) (width 0.2) (layer "F.Cu") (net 4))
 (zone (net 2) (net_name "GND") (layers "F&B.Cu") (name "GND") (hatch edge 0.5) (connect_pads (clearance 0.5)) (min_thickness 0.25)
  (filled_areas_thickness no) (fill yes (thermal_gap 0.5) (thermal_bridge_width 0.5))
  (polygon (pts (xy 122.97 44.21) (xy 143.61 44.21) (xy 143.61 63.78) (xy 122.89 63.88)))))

